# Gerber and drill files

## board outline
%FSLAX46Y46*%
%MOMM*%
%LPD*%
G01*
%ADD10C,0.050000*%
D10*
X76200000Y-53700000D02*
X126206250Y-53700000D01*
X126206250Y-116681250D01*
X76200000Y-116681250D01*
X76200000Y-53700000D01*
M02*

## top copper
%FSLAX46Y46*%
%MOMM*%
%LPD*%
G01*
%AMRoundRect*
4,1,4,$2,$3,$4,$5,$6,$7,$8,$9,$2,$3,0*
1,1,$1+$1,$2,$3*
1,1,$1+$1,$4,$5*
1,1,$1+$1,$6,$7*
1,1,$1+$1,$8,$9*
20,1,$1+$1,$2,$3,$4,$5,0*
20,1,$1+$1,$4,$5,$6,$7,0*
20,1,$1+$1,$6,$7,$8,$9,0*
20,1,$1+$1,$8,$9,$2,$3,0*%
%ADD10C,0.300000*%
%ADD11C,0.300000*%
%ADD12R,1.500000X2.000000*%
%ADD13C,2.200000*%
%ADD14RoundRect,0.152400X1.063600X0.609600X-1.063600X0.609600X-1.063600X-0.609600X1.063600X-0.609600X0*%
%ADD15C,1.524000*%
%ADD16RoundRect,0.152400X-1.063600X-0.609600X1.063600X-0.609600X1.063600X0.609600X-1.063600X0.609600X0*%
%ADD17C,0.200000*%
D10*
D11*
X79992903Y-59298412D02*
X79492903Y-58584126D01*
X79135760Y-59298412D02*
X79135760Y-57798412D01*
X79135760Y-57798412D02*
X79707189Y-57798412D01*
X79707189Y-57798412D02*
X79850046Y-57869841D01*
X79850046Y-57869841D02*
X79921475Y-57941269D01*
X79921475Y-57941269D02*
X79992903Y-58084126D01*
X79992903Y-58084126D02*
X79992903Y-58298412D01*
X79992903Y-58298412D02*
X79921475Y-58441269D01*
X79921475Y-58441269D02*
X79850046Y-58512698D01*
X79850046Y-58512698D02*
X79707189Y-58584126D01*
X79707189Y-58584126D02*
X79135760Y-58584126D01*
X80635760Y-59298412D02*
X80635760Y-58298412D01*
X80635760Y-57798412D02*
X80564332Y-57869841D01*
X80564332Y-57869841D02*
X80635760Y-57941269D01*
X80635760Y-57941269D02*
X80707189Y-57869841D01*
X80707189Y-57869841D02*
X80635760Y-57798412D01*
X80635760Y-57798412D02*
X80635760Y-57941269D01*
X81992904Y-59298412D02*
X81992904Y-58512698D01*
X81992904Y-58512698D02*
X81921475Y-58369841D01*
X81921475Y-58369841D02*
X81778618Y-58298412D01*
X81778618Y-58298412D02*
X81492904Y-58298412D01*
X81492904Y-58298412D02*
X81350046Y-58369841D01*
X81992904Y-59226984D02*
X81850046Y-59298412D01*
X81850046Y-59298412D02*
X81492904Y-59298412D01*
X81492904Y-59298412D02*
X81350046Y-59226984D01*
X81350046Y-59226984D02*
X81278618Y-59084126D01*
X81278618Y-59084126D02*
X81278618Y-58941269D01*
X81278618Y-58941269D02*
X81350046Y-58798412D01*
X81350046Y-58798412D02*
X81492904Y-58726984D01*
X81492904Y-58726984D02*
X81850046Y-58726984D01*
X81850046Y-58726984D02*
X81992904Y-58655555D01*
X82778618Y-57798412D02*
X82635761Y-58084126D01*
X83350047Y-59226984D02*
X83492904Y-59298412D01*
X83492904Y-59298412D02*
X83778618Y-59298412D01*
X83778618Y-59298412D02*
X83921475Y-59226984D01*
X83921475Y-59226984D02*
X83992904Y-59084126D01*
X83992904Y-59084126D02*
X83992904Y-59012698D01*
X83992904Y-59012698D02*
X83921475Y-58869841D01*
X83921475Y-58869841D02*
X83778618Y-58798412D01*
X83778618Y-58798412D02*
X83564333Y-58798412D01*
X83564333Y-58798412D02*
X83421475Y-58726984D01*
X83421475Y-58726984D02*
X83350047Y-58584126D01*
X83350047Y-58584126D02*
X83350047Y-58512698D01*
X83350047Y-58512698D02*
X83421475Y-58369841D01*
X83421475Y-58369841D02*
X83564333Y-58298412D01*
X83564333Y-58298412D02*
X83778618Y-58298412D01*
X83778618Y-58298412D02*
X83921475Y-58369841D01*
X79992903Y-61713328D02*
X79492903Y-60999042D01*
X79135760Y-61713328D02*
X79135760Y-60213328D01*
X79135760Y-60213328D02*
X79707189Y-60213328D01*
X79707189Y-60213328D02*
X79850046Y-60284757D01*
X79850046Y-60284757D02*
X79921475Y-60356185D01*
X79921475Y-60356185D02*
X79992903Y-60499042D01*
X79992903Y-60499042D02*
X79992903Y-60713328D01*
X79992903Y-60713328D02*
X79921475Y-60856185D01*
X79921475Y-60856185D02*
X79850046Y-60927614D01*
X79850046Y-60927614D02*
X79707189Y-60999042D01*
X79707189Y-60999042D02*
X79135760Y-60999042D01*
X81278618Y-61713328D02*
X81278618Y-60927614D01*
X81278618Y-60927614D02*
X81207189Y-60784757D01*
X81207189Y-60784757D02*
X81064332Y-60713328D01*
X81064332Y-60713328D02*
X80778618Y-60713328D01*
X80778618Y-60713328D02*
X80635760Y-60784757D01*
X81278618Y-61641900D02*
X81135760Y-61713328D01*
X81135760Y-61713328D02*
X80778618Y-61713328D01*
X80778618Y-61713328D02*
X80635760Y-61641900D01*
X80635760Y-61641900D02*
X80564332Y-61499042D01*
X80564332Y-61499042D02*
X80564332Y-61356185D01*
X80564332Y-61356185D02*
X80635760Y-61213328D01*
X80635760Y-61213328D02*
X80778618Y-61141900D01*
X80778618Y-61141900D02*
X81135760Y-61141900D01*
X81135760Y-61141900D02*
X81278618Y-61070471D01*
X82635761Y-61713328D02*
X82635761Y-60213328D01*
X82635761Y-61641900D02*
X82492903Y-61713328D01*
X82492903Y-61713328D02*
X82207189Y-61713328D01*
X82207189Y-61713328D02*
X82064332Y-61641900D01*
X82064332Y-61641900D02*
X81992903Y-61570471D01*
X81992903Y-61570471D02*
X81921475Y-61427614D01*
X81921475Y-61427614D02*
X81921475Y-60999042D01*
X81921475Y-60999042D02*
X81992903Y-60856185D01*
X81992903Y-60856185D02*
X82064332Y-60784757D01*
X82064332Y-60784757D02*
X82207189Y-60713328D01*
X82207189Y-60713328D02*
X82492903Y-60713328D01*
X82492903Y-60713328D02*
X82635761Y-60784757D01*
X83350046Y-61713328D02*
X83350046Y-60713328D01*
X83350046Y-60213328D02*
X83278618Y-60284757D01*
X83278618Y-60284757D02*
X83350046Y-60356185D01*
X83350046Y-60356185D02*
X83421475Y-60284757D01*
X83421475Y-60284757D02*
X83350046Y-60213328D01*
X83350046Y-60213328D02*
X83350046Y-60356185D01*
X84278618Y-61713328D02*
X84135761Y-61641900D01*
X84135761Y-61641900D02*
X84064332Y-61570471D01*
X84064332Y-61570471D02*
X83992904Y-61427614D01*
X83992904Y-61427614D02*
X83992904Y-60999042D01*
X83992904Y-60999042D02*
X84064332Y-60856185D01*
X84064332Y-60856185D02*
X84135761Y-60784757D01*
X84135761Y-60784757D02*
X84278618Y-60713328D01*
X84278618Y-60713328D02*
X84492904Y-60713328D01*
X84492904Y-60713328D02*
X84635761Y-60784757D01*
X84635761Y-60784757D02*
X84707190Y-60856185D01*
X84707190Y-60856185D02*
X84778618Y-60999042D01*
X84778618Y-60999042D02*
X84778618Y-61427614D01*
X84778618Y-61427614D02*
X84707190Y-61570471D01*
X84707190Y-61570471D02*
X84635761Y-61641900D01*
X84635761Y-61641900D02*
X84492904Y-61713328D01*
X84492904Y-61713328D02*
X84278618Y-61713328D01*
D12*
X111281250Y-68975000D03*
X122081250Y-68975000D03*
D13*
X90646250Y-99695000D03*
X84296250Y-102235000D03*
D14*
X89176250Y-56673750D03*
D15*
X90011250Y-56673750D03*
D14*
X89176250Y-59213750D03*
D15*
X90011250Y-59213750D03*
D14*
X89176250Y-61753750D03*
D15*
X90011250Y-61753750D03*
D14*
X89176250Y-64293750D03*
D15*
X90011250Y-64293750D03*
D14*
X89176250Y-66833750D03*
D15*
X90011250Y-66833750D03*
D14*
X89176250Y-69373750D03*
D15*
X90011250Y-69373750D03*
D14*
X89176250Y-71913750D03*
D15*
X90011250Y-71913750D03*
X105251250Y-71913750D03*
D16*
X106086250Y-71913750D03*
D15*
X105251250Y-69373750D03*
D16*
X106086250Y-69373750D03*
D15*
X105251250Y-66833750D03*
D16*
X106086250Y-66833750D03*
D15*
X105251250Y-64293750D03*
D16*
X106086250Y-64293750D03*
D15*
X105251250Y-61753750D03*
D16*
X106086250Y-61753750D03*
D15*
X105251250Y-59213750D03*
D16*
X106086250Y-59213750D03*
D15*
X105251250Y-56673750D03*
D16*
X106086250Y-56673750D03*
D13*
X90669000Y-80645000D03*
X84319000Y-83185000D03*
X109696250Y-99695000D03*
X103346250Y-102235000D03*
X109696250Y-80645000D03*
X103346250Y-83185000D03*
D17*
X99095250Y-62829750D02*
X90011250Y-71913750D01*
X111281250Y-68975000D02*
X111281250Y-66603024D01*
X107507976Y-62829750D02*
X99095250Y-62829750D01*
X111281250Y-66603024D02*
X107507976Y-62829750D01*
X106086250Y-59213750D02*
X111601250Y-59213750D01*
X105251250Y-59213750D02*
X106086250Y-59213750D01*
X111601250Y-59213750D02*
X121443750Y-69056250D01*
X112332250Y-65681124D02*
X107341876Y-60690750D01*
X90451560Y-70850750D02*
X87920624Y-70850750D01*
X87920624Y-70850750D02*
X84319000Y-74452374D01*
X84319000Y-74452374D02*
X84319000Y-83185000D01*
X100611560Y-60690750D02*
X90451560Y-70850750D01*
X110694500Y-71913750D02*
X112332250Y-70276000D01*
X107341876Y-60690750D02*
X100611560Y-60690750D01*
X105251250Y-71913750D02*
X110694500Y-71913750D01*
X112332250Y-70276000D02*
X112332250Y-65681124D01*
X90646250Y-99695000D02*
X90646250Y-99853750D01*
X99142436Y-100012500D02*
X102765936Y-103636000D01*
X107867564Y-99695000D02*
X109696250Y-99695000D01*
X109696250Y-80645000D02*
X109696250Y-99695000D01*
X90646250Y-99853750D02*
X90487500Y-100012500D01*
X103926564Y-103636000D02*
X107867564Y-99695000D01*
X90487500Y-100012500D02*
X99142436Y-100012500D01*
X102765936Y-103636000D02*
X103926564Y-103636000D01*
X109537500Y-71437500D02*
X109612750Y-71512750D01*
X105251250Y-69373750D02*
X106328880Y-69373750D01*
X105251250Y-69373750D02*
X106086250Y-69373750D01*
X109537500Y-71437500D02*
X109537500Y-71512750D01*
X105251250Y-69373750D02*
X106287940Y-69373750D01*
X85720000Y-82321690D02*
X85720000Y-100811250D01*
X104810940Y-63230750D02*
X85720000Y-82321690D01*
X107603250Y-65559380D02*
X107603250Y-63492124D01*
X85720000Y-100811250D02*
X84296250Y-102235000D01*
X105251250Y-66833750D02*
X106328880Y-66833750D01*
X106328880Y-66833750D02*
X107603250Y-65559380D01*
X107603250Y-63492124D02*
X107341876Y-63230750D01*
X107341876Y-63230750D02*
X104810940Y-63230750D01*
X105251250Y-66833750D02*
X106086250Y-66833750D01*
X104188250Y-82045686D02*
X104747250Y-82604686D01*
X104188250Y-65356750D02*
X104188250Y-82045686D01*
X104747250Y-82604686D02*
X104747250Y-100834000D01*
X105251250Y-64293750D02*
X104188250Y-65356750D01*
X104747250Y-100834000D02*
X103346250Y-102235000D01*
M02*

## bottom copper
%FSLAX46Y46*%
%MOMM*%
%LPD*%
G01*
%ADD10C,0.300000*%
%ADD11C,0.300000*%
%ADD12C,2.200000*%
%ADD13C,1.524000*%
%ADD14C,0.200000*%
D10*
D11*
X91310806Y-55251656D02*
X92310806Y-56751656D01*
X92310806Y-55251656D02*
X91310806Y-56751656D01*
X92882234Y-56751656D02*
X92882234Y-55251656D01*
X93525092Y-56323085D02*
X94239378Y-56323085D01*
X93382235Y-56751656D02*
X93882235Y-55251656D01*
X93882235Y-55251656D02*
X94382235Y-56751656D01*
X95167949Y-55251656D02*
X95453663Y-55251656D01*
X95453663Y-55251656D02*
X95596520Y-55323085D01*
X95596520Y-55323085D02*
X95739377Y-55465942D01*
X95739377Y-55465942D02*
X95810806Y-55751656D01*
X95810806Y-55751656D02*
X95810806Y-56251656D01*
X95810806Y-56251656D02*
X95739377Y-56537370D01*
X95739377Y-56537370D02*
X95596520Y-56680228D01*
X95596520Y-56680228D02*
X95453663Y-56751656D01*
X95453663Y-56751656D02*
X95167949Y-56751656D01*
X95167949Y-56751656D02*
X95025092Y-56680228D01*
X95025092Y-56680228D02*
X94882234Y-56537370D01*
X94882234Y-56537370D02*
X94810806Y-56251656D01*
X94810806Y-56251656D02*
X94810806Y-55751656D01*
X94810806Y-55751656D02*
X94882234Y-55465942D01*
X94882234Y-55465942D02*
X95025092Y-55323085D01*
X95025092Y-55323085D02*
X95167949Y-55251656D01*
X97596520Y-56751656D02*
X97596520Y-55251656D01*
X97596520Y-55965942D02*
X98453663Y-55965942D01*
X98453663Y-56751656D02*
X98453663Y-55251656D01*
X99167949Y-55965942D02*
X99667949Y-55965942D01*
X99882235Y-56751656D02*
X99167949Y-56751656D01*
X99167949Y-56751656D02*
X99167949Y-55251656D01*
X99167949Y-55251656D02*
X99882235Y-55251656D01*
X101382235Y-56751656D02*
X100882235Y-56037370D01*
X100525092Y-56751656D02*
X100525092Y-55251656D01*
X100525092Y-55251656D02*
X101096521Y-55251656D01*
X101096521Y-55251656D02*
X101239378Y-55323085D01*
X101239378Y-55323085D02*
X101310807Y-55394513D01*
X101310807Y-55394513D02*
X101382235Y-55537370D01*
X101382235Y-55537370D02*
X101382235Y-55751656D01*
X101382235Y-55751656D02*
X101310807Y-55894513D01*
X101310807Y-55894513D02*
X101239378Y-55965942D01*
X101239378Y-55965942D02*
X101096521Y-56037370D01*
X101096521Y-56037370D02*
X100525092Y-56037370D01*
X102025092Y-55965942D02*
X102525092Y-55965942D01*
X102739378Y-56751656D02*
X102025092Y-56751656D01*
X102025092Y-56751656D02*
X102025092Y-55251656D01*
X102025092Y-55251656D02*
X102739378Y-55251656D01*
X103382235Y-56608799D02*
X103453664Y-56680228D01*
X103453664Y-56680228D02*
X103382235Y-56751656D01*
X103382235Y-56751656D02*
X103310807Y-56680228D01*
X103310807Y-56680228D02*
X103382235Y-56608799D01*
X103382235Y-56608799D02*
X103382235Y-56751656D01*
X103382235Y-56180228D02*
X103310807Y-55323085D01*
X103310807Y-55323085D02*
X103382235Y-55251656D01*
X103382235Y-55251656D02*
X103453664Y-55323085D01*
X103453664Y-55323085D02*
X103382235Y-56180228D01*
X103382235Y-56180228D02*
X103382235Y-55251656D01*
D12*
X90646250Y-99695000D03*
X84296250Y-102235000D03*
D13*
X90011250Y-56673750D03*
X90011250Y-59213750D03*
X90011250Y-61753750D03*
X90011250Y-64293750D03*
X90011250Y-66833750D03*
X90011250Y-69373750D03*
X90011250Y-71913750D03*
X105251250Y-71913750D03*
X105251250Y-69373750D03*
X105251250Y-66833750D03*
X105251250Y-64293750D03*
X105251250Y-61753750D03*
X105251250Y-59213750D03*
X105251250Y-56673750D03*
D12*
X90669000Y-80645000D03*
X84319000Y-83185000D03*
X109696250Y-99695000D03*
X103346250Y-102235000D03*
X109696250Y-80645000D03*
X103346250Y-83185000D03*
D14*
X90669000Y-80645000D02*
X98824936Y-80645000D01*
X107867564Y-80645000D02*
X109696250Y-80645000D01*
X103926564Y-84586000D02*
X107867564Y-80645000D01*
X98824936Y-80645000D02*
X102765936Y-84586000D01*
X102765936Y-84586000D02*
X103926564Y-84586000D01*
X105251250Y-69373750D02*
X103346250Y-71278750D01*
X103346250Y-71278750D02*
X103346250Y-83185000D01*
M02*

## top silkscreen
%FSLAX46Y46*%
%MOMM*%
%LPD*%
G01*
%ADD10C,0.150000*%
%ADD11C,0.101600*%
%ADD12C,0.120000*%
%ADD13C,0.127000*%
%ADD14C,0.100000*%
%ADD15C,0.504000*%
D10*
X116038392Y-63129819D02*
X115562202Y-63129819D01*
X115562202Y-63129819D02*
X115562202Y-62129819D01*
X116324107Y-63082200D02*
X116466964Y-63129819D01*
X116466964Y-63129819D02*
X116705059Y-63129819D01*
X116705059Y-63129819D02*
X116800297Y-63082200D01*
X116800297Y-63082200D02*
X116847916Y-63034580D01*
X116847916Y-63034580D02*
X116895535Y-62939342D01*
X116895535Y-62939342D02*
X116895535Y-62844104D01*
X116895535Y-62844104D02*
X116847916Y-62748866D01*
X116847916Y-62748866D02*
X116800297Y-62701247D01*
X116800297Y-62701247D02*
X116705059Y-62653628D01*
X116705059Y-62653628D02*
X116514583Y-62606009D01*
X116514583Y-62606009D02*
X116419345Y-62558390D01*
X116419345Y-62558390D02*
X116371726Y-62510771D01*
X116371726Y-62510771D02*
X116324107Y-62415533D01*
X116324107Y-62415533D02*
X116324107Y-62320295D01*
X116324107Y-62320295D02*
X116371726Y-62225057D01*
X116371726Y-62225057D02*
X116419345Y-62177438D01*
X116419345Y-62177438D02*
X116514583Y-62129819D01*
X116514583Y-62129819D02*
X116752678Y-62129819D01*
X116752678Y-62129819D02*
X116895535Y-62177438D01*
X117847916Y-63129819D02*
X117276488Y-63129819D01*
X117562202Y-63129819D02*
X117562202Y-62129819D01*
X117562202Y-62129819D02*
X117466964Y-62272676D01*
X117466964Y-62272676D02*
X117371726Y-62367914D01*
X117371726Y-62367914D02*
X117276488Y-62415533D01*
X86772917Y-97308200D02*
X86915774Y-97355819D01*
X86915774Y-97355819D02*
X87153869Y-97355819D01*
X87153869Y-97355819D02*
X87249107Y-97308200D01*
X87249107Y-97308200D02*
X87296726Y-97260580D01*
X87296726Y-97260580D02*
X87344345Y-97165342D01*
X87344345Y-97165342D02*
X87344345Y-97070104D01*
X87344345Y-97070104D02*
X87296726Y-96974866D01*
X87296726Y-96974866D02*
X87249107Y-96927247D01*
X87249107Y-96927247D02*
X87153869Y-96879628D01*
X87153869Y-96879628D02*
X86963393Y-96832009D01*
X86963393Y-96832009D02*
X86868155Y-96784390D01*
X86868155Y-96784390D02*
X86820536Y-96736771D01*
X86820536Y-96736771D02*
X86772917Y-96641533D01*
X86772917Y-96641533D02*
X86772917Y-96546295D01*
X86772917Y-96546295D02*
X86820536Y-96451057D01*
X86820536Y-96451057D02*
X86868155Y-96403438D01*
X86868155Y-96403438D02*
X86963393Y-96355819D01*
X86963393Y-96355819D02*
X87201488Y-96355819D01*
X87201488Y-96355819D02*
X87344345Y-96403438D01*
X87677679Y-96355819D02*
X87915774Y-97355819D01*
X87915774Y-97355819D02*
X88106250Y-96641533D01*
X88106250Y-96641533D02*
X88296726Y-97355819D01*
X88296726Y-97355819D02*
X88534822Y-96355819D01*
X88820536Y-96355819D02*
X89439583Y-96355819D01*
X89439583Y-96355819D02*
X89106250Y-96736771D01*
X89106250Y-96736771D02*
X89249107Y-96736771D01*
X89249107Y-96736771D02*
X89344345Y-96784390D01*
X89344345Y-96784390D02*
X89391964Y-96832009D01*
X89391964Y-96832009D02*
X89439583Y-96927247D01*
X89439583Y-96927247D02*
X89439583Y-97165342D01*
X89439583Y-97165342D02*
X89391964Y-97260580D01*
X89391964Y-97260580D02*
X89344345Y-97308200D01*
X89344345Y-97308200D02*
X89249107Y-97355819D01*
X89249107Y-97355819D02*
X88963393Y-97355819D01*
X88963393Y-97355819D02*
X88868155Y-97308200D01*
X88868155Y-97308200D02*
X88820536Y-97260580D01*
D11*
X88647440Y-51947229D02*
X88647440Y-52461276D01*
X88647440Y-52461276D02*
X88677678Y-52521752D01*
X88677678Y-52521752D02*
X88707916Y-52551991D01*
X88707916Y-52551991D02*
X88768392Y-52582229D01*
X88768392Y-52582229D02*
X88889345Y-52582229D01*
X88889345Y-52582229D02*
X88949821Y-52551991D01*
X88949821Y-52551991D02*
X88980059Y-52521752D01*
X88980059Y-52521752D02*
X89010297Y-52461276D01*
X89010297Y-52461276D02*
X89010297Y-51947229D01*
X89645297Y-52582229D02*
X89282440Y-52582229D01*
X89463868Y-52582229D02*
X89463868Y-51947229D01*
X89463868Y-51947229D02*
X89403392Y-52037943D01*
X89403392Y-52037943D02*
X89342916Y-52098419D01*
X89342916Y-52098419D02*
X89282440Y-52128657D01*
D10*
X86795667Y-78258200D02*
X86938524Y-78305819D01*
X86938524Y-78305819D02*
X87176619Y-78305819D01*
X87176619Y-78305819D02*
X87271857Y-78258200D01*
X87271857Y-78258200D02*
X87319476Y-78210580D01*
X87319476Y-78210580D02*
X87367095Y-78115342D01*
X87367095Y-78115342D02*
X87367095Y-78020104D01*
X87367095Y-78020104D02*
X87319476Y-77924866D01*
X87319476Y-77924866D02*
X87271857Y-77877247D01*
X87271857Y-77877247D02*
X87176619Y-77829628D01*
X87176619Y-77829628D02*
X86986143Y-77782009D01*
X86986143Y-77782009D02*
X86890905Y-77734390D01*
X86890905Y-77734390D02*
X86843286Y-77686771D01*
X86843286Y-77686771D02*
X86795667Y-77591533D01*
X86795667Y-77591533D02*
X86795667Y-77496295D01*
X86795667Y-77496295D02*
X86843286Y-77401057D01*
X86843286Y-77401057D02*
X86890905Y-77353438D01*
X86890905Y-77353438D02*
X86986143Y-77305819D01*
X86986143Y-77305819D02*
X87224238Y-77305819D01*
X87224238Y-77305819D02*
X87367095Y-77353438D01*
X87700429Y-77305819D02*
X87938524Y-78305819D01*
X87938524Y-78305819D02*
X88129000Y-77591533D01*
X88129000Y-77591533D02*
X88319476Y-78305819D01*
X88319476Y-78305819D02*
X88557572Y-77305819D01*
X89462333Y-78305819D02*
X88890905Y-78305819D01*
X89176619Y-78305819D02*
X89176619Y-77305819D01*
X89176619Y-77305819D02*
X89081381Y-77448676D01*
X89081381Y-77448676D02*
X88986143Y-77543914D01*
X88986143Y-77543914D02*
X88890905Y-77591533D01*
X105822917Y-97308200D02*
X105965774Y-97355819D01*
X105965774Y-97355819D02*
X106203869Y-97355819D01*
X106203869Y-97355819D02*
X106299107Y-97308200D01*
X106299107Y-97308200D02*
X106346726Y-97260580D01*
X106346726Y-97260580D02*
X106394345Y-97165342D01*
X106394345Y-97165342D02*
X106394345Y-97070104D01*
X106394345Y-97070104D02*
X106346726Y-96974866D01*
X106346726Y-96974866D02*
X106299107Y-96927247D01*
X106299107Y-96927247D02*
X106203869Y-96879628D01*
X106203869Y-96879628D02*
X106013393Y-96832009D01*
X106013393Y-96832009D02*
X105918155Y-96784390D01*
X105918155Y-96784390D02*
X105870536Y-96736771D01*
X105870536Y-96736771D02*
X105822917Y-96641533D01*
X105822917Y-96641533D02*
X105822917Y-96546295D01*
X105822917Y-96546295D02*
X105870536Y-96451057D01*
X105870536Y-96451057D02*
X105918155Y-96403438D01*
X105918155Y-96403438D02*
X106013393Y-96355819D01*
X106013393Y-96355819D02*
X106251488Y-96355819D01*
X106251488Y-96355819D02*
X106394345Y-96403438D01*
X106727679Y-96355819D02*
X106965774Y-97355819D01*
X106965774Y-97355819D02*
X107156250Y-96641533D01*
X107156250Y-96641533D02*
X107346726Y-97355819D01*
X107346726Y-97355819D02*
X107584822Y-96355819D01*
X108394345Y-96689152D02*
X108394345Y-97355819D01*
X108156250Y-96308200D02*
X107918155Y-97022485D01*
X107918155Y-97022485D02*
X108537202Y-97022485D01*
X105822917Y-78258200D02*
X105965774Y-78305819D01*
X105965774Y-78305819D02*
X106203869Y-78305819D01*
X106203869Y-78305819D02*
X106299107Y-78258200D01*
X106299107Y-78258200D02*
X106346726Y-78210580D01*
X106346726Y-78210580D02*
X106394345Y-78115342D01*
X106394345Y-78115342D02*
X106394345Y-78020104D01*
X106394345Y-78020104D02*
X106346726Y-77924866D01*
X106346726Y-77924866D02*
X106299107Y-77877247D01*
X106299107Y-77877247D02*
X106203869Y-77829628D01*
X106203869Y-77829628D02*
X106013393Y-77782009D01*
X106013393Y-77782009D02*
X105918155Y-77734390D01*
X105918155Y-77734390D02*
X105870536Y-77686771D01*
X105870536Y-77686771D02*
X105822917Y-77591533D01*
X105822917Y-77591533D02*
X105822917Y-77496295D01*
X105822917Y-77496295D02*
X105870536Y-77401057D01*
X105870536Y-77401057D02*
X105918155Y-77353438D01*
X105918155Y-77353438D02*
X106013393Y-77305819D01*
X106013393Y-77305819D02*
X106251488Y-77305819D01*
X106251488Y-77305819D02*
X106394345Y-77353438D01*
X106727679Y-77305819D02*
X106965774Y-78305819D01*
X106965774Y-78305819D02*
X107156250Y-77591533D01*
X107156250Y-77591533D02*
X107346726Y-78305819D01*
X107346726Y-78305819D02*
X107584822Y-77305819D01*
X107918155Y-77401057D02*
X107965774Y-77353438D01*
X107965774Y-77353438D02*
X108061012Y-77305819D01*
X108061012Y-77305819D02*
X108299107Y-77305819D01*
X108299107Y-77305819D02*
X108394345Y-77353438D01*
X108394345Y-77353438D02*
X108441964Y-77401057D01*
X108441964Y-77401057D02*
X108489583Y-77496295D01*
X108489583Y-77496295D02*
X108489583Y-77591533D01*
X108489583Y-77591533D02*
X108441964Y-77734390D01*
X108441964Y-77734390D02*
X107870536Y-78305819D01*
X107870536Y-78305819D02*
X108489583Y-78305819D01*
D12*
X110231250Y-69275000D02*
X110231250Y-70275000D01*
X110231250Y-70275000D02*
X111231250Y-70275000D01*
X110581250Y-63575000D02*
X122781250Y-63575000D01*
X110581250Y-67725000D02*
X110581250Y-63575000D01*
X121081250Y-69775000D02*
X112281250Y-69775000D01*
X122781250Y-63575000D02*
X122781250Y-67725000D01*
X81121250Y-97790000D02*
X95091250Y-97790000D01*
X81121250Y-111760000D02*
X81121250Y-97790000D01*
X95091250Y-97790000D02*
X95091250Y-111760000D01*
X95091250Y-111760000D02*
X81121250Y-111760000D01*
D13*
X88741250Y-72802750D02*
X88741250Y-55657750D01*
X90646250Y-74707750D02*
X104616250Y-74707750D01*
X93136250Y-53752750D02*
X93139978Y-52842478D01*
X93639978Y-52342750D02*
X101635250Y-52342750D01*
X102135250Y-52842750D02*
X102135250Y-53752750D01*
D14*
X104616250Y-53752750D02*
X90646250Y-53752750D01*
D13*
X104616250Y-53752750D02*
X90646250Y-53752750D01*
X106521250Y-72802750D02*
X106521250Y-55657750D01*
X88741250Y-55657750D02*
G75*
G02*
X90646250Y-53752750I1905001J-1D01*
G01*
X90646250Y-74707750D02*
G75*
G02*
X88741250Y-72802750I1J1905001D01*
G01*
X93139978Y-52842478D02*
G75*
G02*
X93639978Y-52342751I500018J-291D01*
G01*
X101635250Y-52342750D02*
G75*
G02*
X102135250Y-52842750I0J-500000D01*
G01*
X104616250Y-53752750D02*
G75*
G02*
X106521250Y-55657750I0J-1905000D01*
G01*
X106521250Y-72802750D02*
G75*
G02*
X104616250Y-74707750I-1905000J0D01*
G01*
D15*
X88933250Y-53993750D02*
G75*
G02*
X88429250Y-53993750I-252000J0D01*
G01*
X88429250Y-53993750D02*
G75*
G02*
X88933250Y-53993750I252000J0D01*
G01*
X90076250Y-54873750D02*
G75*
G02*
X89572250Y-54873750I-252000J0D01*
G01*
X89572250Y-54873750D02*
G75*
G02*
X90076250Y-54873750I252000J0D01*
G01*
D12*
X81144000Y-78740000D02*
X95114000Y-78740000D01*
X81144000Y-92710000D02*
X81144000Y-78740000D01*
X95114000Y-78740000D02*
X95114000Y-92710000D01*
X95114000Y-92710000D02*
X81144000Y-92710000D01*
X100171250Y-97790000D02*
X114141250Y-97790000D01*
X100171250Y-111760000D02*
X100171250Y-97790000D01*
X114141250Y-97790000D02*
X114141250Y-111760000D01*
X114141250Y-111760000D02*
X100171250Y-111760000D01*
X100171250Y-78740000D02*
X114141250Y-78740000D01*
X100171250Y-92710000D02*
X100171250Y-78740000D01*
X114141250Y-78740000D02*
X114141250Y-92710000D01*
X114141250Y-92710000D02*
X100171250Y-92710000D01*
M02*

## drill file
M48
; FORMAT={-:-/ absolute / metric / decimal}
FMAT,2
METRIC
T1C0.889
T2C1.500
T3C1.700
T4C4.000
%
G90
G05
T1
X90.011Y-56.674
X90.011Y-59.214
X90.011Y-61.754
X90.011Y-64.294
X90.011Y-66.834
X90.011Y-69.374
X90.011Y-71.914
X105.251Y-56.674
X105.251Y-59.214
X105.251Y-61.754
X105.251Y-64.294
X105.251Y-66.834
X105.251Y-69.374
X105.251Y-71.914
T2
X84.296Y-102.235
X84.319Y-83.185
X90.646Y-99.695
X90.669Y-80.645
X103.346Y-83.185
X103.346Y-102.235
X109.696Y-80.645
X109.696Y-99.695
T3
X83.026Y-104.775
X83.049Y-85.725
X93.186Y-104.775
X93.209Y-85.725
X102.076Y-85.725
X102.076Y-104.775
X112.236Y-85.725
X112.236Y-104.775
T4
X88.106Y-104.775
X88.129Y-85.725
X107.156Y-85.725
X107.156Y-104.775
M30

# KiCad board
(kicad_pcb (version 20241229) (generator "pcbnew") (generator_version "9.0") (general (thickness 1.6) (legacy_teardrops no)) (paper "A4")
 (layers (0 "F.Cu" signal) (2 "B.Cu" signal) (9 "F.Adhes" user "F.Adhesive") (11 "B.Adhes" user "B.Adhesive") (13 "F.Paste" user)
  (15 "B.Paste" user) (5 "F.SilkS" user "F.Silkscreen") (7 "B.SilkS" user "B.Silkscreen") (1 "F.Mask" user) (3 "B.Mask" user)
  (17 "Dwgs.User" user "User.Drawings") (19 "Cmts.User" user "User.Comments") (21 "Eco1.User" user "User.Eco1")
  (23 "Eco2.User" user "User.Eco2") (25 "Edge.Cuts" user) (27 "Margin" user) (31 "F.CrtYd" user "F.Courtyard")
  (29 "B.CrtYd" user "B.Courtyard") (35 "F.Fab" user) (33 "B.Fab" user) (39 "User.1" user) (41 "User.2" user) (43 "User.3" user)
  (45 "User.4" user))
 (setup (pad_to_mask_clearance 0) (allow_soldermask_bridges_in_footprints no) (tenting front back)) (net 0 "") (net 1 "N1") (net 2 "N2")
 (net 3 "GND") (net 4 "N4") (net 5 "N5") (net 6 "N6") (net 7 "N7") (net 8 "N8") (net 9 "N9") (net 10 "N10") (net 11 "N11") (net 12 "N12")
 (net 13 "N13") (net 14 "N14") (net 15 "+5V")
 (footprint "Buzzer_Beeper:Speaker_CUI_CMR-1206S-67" (layer "F.Cu") (at 116.68125 66.675)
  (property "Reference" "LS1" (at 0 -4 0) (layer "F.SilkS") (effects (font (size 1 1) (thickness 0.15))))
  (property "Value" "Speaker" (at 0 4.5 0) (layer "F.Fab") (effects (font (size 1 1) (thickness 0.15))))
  (fp_line (start -6.45 2.6) (end -6.45 3.6) (stroke (width 0.12) (type solid)) (layer "F.SilkS"))
  (fp_line (start -6.45 3.6) (end -5.45 3.6) (stroke (width 0.12) (type solid)) (layer "F.SilkS"))
  (fp_line (start -6.1 -3.1) (end 6.1 -3.1) (stroke (width 0.12) (type solid)) (layer "F.SilkS"))
  (fp_line (start -6.1 1.05) (end -6.1 -3.1) (stroke (width 0.12) (type solid)) (layer "F.SilkS"))
  (fp_line (start 4.4 3.1) (end -4.4 3.1) (stroke (width 0.12) (type solid)) (layer "F.SilkS"))
  (fp_line (start 6.1 -3.1) (end 6.1 1.05) (stroke (width 0.12) (type solid)) (layer "F.SilkS"))
  (pad "1" smd rect (at -5.4 2.3 180) (size 1.5 2) (layers "F.Cu" "F.Mask") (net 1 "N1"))
  (pad "2" smd rect (at 5.4 2.3 180) (size 1.5 2) (layers "F.Cu" "F.Mask") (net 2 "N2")))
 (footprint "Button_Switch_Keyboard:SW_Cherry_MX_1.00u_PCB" (layer "F.Cu") (at 90.64625 99.695)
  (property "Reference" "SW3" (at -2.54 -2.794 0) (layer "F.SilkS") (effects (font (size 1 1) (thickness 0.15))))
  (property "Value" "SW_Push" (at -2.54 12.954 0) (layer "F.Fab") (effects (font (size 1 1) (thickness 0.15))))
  (fp_line (start -9.525 -1.905) (end 4.445 -1.905) (stroke (width 0.12) (type solid)) (layer "F.SilkS"))
  (fp_line (start -9.525 12.065) (end -9.525 -1.905) (stroke (width 0.12) (type solid)) (layer "F.SilkS"))
  (fp_line (start 4.445 -1.905) (end 4.445 12.065) (stroke (width 0.12) (type solid)) (layer "F.SilkS"))
  (fp_line (start 4.445 12.065) (end -9.525 12.065) (stroke (width 0.12) (type solid)) (layer "F.SilkS"))
  (pad "" np_thru_hole circle (at -7.62 5.08) (size 1.7 1.7) (drill 1.7) (layers "*.Cu" "*.Mask"))
  (pad "" np_thru_hole circle (at -2.54 5.08) (size 4 4) (drill 4) (layers "*.Cu" "*.Mask"))
  (pad "" np_thru_hole circle (at 2.54 5.08) (size 1.7 1.7) (drill 1.7) (layers "*.Cu" "*.Mask"))
  (pad "1" thru_hole circle (at 0 0) (size 2.2 2.2) (drill 1.5) (layers "*.Cu" "*.Mask") (remove_unused_layers no) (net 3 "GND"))
  (pad "2" thru_hole circle (at -6.35 2.54) (size 2.2 2.2) (drill 1.5) (layers "*.Cu" "*.Mask") (remove_unused_layers no) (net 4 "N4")))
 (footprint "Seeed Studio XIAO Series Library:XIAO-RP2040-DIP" (layer "F.Cu") (at 97.63125 64.29375)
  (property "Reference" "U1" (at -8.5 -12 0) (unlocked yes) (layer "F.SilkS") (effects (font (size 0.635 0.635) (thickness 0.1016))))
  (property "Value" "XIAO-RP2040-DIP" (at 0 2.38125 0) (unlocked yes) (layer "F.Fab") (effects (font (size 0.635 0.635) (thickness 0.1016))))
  (fp_line (start -8.89 8.509) (end -8.89 -8.636) (stroke (width 0.127) (type solid)) (layer "F.SilkS"))
  (fp_line (start -6.985 10.414) (end 6.985 10.414) (stroke (width 0.127) (type solid)) (layer "F.SilkS"))
  (fp_line (start -4.495 -10.541) (end -4.491272 -11.451272) (stroke (width 0.127) (type solid)) (layer "F.SilkS"))
  (fp_line (start -3.991272 -11.951) (end 4.004 -11.951) (stroke (width 0.127) (type solid)) (layer "F.SilkS"))
  (fp_line (start 4.504 -11.451) (end 4.504 -10.541) (stroke (width 0.127) (type solid)) (layer "F.SilkS"))
  (fp_line (start 6.985 -10.541) (end -6.985 -10.541) (stroke (width 0.1) (type solid)) (layer "F.SilkS"))
  (fp_line (start 6.985 -10.541) (end -6.985 -10.541) (stroke (width 0.127) (type solid)) (layer "F.SilkS"))
  (fp_line (start 8.89 8.509) (end 8.89 -8.636) (stroke (width 0.127) (type solid)) (layer "F.SilkS"))
  (fp_arc (start -8.89 -8.636) (mid -8.332038 -9.983038) (end -6.985 -10.541) (stroke (width 0.127) (type solid)) (layer "F.SilkS"))
  (fp_arc (start -6.985 10.414) (mid -8.332038 9.856038) (end -8.89 8.509) (stroke (width 0.127) (type solid)) (layer "F.SilkS"))
  (fp_arc (start -4.491272 -11.451272) (mid -4.344728 -11.80464) (end -3.991272 -11.951) (stroke (width 0.127) (type default))
   (layer "F.SilkS"))
  (fp_arc (start 4.004 -11.951) (mid 4.357553 -11.804553) (end 4.504 -11.451) (stroke (width 0.127) (type default)) (layer "F.SilkS"))
  (fp_arc (start 6.985 -10.541) (mid 8.332038 -9.983038) (end 8.89 -8.636) (stroke (width 0.127) (type solid)) (layer "F.SilkS"))
  (fp_arc (start 8.89 8.509) (mid 8.332038 9.856038) (end 6.985 10.414) (stroke (width 0.127) (type solid)) (layer "F.SilkS"))
  (fp_circle (center -8.95 -10.3) (end -8.95 -10.554) (stroke (width 0.5) (type solid)) (fill yes) (layer "F.SilkS"))
  (fp_circle (center -7.807 -9.42) (end -7.807 -9.674) (stroke (width 0.5) (type solid)) (fill yes) (layer "F.SilkS"))
  (pad "1" smd roundrect (at -8.455 -7.62 180) (size 2.432 1.524) (layers "F.Cu" "F.Mask") (roundrect_rratio 0.1) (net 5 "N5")
   (thermal_bridge_angle 45))
  (pad "1" thru_hole circle (at -7.62 -7.62 180) (size 1.524 1.524) (drill 0.889) (layers "*.Cu" "*.Mask") (remove_unused_layers no)
   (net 5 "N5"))
  (pad "2" smd roundrect (at -8.455 -5.08 180) (size 2.432 1.524) (layers "F.Cu" "F.Mask") (roundrect_rratio 0.1) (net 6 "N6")
   (thermal_bridge_angle 45))
  (pad "2" thru_hole circle (at -7.62 -5.08 180) (size 1.524 1.524) (drill 0.889) (layers "*.Cu" "*.Mask") (remove_unused_layers no)
   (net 6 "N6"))
  (pad "3" smd roundrect (at -8.455 -2.54 180) (size 2.432 1.524) (layers "F.Cu" "F.Mask") (roundrect_rratio 0.1) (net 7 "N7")
   (thermal_bridge_angle 45))
  (pad "3" thru_hole circle (at -7.62 -2.54 180) (size 1.524 1.524) (drill 0.889) (layers "*.Cu" "*.Mask") (remove_unused_layers no)
   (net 7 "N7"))
  (pad "4" smd roundrect (at -8.455 0 180) (size 2.432 1.524) (layers "F.Cu" "F.Mask") (roundrect_rratio 0.1) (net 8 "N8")
   (thermal_bridge_angle 45))
  (pad "4" thru_hole circle (at -7.62 0 180) (size 1.524 1.524) (drill 0.889) (layers "*.Cu" "*.Mask") (remove_unused_layers no)
   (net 8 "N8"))
  (pad "5" smd roundrect (at -8.455 2.54 180) (size 2.432 1.524) (layers "F.Cu" "F.Mask") (roundrect_rratio 0.1) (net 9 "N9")
   (thermal_bridge_angle 45))
  (pad "5" thru_hole circle (at -7.62 2.54 180) (size 1.524 1.524) (drill 0.889) (layers "*.Cu" "*.Mask") (remove_unused_layers no)
   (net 9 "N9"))
  (pad "6" smd roundrect (at -8.455 5.08 180) (size 2.432 1.524) (layers "F.Cu" "F.Mask") (roundrect_rratio 0.1) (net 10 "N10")
   (thermal_bridge_angle 45))
  (pad "6" thru_hole circle (at -7.62 5.08 180) (size 1.524 1.524) (drill 0.889) (layers "*.Cu" "*.Mask") (remove_unused_layers no)
   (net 10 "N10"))
  (pad "7" smd roundrect (at -8.455 7.62 180) (size 2.432 1.524) (layers "F.Cu" "F.Mask") (roundrect_rratio 0.1) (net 1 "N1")
   (thermal_bridge_angle 45))
  (pad "7" thru_hole circle (at -7.62 7.62 180) (size 1.524 1.524) (drill 0.889) (layers "*.Cu" "*.Mask") (remove_unused_layers no)
   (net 1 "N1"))
  (pad "8" thru_hole circle (at 7.62 7.62) (size 1.524 1.524) (drill 0.889) (layers "*.Cu" "*.Mask") (remove_unused_layers no)
   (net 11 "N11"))
  (pad "8" smd roundrect (at 8.455 7.62) (size 2.432 1.524) (layers "F.Cu" "F.Mask") (roundrect_rratio 0.1) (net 11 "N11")
   (thermal_bridge_angle 45))
  (pad "9" thru_hole circle (at 7.62 5.08) (size 1.524 1.524) (drill 0.889) (layers "*.Cu" "*.Mask") (remove_unused_layers no)
   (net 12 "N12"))
  (pad "9" smd roundrect (at 8.455 5.08) (size 2.432 1.524) (layers "F.Cu" "F.Mask") (roundrect_rratio 0.1) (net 12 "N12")
   (thermal_bridge_angle 45))
  (pad "10" thru_hole circle (at 7.62 2.54) (size 1.524 1.524) (drill 0.889) (layers "*.Cu" "*.Mask") (remove_unused_layers no) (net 4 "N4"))
  (pad "10" smd roundrect (at 8.455 2.54) (size 2.432 1.524) (layers "F.Cu" "F.Mask") (roundrect_rratio 0.1) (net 4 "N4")
   (thermal_bridge_angle 45))
  (pad "11" thru_hole circle (at 7.62 0) (size 1.524 1.524) (drill 0.889) (layers "*.Cu" "*.Mask") (remove_unused_layers no) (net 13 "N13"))
  (pad "11" smd roundrect (at 8.455 0) (size 2.432 1.524) (layers "F.Cu" "F.Mask") (roundrect_rratio 0.1) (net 13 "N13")
   (thermal_bridge_angle 45))
  (pad "12" thru_hole circle (at 7.62 -2.54) (size 1.524 1.524) (drill 0.889) (layers "*.Cu" "*.Mask") (remove_unused_layers no)
   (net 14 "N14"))
  (pad "12" smd roundrect (at 8.455 -2.54) (size 2.432 1.524) (layers "F.Cu" "F.Mask") (roundrect_rratio 0.1) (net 14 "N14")
   (thermal_bridge_angle 45))
  (pad "13" thru_hole circle (at 7.62 -5.08) (size 1.524 1.524) (drill 0.889) (layers "*.Cu" "*.Mask") (remove_unused_layers no)
   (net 2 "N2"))
  (pad "13" smd roundrect (at 8.455 -5.08) (size 2.432 1.524) (layers "F.Cu" "F.Mask") (roundrect_rratio 0.1) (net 2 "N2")
   (thermal_bridge_angle 45))
  (pad "14" thru_hole circle (at 7.62 -7.62) (size 1.524 1.524) (drill 0.889) (layers "*.Cu" "*.Mask") (remove_unused_layers no)
   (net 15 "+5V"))
  (pad "14" smd roundrect (at 8.455 -7.62) (size 2.432 1.524) (layers "F.Cu" "F.Mask") (roundrect_rratio 0.1) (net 15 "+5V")
   (thermal_bridge_angle 45)))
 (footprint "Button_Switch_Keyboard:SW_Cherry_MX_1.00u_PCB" (layer "F.Cu") (at 90.669 80.645)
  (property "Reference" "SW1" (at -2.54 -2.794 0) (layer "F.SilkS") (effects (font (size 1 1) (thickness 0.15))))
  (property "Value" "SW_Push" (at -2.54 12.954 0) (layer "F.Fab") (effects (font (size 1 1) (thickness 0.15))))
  (fp_line (start -9.525 -1.905) (end 4.445 -1.905) (stroke (width 0.12) (type solid)) (layer "F.SilkS"))
  (fp_line (start -9.525 12.065) (end -9.525 -1.905) (stroke (width 0.12) (type solid)) (layer "F.SilkS"))
  (fp_line (start 4.445 -1.905) (end 4.445 12.065) (stroke (width 0.12) (type solid)) (layer "F.SilkS"))
  (fp_line (start 4.445 12.065) (end -9.525 12.065) (stroke (width 0.12) (type solid)) (layer "F.SilkS"))
  (pad "" np_thru_hole circle (at -7.62 5.08) (size 1.7 1.7) (drill 1.7) (layers "*.Cu" "*.Mask"))
  (pad "" np_thru_hole circle (at -2.54 5.08) (size 4 4) (drill 4) (layers "*.Cu" "*.Mask"))
  (pad "" np_thru_hole circle (at 2.54 5.08) (size 1.7 1.7) (drill 1.7) (layers "*.Cu" "*.Mask"))
  (pad "1" thru_hole circle (at 0 0) (size 2.2 2.2) (drill 1.5) (layers "*.Cu" "*.Mask") (remove_unused_layers no) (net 3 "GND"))
  (pad "2" thru_hole circle (at -6.35 2.54) (size 2.2 2.2) (drill 1.5) (layers "*.Cu" "*.Mask") (remove_unused_layers no) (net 11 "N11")))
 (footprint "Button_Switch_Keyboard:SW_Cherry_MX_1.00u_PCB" (layer "F.Cu") (at 109.69625 99.695)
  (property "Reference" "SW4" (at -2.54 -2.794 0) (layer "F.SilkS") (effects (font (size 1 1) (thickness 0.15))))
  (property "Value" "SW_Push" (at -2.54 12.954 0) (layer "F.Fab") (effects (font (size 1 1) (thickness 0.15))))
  (fp_line (start -9.525 -1.905) (end 4.445 -1.905) (stroke (width 0.12) (type solid)) (layer "F.SilkS"))
  (fp_line (start -9.525 12.065) (end -9.525 -1.905) (stroke (width 0.12) (type solid)) (layer "F.SilkS"))
  (fp_line (start 4.445 -1.905) (end 4.445 12.065) (stroke (width 0.12) (type solid)) (layer "F.SilkS"))
  (fp_line (start 4.445 12.065) (end -9.525 12.065) (stroke (width 0.12) (type solid)) (layer "F.SilkS"))
  (pad "" np_thru_hole circle (at -7.62 5.08) (size 1.7 1.7) (drill 1.7) (layers "*.Cu" "*.Mask"))
  (pad "" np_thru_hole circle (at -2.54 5.08) (size 4 4) (drill 4) (layers "*.Cu" "*.Mask"))
  (pad "" np_thru_hole circle (at 2.54 5.08) (size 1.7 1.7) (drill 1.7) (layers "*.Cu" "*.Mask"))
  (pad "1" thru_hole circle (at 0 0) (size 2.2 2.2) (drill 1.5) (layers "*.Cu" "*.Mask") (remove_unused_layers no) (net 3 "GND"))
  (pad "2" thru_hole circle (at -6.35 2.54) (size 2.2 2.2) (drill 1.5) (layers "*.Cu" "*.Mask") (remove_unused_layers no) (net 13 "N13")))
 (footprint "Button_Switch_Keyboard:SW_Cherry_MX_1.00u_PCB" (layer "F.Cu") (at 109.69625 80.645)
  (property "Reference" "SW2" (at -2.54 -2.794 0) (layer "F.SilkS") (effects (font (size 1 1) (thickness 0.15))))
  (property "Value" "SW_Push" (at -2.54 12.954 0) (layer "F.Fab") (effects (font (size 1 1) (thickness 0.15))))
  (fp_line (start -9.525 -1.905) (end 4.445 -1.905) (stroke (width 0.12) (type solid)) (layer "F.SilkS"))
  (fp_line (start -9.525 12.065) (end -9.525 -1.905) (stroke (width 0.12) (type solid)) (layer "F.SilkS"))
  (fp_line (start 4.445 -1.905) (end 4.445 12.065) (stroke (width 0.12) (type solid)) (layer "F.SilkS"))
  (fp_line (start 4.445 12.065) (end -9.525 12.065) (stroke (width 0.12) (type solid)) (layer "F.SilkS"))
  (pad "" np_thru_hole circle (at -7.62 5.08) (size 1.7 1.7) (drill 1.7) (layers "*.Cu" "*.Mask"))
  (pad "" np_thru_hole circle (at -2.54 5.08) (size 4 4) (drill 4) (layers "*.Cu" "*.Mask"))
  (pad "" np_thru_hole circle (at 2.54 5.08) (size 1.7 1.7) (drill 1.7) (layers "*.Cu" "*.Mask"))
  (pad "1" thru_hole circle (at 0 0) (size 2.2 2.2) (drill 1.5) (layers "*.Cu" "*.Mask") (remove_unused_layers no) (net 3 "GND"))
  (pad "2" thru_hole circle (at -6.35 2.54) (size 2.2 2.2) (drill 1.5) (layers "*.Cu" "*.Mask") (remove_unused_layers no) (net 12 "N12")))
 (gr_rect (start 76.2 53.7) (end 126.20625 116.68125) (stroke (width 0.05) (type solid)) (fill no) (layer "Edge.Cuts"))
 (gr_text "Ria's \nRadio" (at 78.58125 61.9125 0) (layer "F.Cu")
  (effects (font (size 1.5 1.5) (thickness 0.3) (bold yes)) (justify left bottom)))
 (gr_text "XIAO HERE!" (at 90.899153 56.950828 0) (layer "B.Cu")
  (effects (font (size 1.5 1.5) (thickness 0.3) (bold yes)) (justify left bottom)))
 (segment (start 99.09525 62.82975) (end 90.01125 71.91375) (width 0.2) (layer "F.Cu") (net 1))
 (segment (start 111.28125 68.975) (end 111.28125 66.603024) (width 0.2) (layer "F.Cu") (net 1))
 (segment (start 107.507976 62.82975) (end 99.09525 62.82975) (width 0.2) (layer "F.Cu") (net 1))
 (segment (start 111.28125 66.603024) (end 107.507976 62.82975) (width 0.2) (layer "F.Cu") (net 1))
 (segment (start 106.08625 59.21375) (end 111.60125 59.21375) (width 0.2) (layer "F.Cu") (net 2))
 (segment (start 105.25125 59.21375) (end 106.08625 59.21375) (width 0.2) (layer "F.Cu") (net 2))
 (segment (start 111.60125 59.21375) (end 121.44375 69.05625) (width 0.2) (layer "F.Cu") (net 2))
 (segment (start 112.33225 65.681124) (end 107.341876 60.69075) (width 0.2) (layer "F.Cu") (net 11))
 (segment (start 90.45156 70.85075) (end 87.920624 70.85075) (width 0.2) (layer "F.Cu") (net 11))
 (segment (start 87.920624 70.85075) (end 84.319 74.452374) (width 0.2) (layer "F.Cu") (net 11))
 (segment (start 84.319 74.452374) (end 84.319 83.185) (width 0.2) (layer "F.Cu") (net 11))
 (segment (start 100.61156 60.69075) (end 90.45156 70.85075) (width 0.2) (layer "F.Cu") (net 11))
 (segment (start 110.6945 71.91375) (end 112.33225 70.276) (width 0.2) (layer "F.Cu") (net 11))
 (segment (start 107.341876 60.69075) (end 100.61156 60.69075) (width 0.2) (layer "F.Cu") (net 11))
 (segment (start 105.25125 71.91375) (end 110.6945 71.91375) (width 0.2) (layer "F.Cu") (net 11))
 (segment (start 112.33225 70.276) (end 112.33225 65.681124) (width 0.2) (layer "F.Cu") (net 11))
 (segment (start 90.64625 99.695) (end 90.64625 99.85375) (width 0.2) (layer "F.Cu") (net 3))
 (segment (start 99.142436 100.0125) (end 102.765936 103.636) (width 0.2) (layer "F.Cu") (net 3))
 (segment (start 107.867564 99.695) (end 109.69625 99.695) (width 0.2) (layer "F.Cu") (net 3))
 (segment (start 109.69625 80.645) (end 109.69625 99.695) (width 0.2) (layer "F.Cu") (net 3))
 (segment (start 90.64625 99.85375) (end 90.4875 100.0125) (width 0.2) (layer "F.Cu") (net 3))
 (segment (start 103.926564 103.636) (end 107.867564 99.695) (width 0.2) (layer "F.Cu") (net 3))
 (segment (start 90.4875 100.0125) (end 99.142436 100.0125) (width 0.2) (layer "F.Cu") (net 3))
 (segment (start 102.765936 103.636) (end 103.926564 103.636) (width 0.2) (layer "F.Cu") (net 3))
 (segment (start 90.669 80.645) (end 98.824936 80.645) (width 0.2) (layer "B.Cu") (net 3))
 (segment (start 107.867564 80.645) (end 109.69625 80.645) (width 0.2) (layer "B.Cu") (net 3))
 (segment (start 103.926564 84.586) (end 107.867564 80.645) (width 0.2) (layer "B.Cu") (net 3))
 (segment (start 98.824936 80.645) (end 102.765936 84.586) (width 0.2) (layer "B.Cu") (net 3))
 (segment (start 102.765936 84.586) (end 103.926564 84.586) (width 0.2) (layer "B.Cu") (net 3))
 (segment (start 109.5375 71.4375) (end 109.61275 71.51275) (width 0.2) (layer "F.Cu") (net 12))
 (segment (start 105.25125 69.37375) (end 106.32888 69.37375) (width 0.2) (layer "F.Cu") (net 12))
 (segment (start 105.25125 69.37375) (end 106.08625 69.37375) (width 0.2) (layer "F.Cu") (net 12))
 (segment (start 109.5375 71.4375) (end 109.5375 71.51275) (width 0.2) (layer "F.Cu") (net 12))
 (segment (start 105.25125 69.37375) (end 106.28794 69.37375) (width 0.2) (layer "F.Cu") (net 12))
 (segment (start 105.25125 69.37375) (end 103.34625 71.27875) (width 0.2) (layer "B.Cu") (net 12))
 (segment (start 103.34625 71.27875) (end 103.34625 83.185) (width 0.2) (layer "B.Cu") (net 12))
 (segment (start 85.72 82.32169) (end 85.72 100.81125) (width 0.2) (layer "F.Cu") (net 4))
 (segment (start 104.81094 63.23075) (end 85.72 82.32169) (width 0.2) (layer "F.Cu") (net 4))
 (segment (start 107.60325 65.55938) (end 107.60325 63.492124) (width 0.2) (layer "F.Cu") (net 4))
 (segment (start 85.72 100.81125) (end 84.29625 102.235) (width 0.2) (layer "F.Cu") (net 4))
 (segment (start 105.25125 66.83375) (end 106.32888 66.83375) (width 0.2) (layer "F.Cu") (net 4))
 (segment (start 106.32888 66.83375) (end 107.60325 65.55938) (width 0.2) (layer "F.Cu") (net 4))
 (segment (start 107.60325 63.492124) (end 107.341876 63.23075) (width 0.2) (layer "F.Cu") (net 4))
 (segment (start 107.341876 63.23075) (end 104.81094 63.23075) (width 0.2) (layer "F.Cu") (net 4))
 (segment (start 105.25125 66.83375) (end 106.08625 66.83375) (width 0.2) (layer "F.Cu") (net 4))
 (segment (start 104.18825 82.045686) (end 104.74725 82.604686) (width 0.2) (layer "F.Cu") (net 13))
 (segment (start 104.18825 65.35675) (end 104.18825 82.045686) (width 0.2) (layer "F.Cu") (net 13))
 (segment (start 104.74725 82.604686) (end 104.74725 100.834) (width 0.2) (layer "F.Cu") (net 13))
 (segment (start 105.25125 64.29375) (end 104.18825 65.35675) (width 0.2) (layer "F.Cu") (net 13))
 (segment (start 104.74725 100.834) (end 103.34625 102.235) (width 0.2) (layer "F.Cu") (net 13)))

